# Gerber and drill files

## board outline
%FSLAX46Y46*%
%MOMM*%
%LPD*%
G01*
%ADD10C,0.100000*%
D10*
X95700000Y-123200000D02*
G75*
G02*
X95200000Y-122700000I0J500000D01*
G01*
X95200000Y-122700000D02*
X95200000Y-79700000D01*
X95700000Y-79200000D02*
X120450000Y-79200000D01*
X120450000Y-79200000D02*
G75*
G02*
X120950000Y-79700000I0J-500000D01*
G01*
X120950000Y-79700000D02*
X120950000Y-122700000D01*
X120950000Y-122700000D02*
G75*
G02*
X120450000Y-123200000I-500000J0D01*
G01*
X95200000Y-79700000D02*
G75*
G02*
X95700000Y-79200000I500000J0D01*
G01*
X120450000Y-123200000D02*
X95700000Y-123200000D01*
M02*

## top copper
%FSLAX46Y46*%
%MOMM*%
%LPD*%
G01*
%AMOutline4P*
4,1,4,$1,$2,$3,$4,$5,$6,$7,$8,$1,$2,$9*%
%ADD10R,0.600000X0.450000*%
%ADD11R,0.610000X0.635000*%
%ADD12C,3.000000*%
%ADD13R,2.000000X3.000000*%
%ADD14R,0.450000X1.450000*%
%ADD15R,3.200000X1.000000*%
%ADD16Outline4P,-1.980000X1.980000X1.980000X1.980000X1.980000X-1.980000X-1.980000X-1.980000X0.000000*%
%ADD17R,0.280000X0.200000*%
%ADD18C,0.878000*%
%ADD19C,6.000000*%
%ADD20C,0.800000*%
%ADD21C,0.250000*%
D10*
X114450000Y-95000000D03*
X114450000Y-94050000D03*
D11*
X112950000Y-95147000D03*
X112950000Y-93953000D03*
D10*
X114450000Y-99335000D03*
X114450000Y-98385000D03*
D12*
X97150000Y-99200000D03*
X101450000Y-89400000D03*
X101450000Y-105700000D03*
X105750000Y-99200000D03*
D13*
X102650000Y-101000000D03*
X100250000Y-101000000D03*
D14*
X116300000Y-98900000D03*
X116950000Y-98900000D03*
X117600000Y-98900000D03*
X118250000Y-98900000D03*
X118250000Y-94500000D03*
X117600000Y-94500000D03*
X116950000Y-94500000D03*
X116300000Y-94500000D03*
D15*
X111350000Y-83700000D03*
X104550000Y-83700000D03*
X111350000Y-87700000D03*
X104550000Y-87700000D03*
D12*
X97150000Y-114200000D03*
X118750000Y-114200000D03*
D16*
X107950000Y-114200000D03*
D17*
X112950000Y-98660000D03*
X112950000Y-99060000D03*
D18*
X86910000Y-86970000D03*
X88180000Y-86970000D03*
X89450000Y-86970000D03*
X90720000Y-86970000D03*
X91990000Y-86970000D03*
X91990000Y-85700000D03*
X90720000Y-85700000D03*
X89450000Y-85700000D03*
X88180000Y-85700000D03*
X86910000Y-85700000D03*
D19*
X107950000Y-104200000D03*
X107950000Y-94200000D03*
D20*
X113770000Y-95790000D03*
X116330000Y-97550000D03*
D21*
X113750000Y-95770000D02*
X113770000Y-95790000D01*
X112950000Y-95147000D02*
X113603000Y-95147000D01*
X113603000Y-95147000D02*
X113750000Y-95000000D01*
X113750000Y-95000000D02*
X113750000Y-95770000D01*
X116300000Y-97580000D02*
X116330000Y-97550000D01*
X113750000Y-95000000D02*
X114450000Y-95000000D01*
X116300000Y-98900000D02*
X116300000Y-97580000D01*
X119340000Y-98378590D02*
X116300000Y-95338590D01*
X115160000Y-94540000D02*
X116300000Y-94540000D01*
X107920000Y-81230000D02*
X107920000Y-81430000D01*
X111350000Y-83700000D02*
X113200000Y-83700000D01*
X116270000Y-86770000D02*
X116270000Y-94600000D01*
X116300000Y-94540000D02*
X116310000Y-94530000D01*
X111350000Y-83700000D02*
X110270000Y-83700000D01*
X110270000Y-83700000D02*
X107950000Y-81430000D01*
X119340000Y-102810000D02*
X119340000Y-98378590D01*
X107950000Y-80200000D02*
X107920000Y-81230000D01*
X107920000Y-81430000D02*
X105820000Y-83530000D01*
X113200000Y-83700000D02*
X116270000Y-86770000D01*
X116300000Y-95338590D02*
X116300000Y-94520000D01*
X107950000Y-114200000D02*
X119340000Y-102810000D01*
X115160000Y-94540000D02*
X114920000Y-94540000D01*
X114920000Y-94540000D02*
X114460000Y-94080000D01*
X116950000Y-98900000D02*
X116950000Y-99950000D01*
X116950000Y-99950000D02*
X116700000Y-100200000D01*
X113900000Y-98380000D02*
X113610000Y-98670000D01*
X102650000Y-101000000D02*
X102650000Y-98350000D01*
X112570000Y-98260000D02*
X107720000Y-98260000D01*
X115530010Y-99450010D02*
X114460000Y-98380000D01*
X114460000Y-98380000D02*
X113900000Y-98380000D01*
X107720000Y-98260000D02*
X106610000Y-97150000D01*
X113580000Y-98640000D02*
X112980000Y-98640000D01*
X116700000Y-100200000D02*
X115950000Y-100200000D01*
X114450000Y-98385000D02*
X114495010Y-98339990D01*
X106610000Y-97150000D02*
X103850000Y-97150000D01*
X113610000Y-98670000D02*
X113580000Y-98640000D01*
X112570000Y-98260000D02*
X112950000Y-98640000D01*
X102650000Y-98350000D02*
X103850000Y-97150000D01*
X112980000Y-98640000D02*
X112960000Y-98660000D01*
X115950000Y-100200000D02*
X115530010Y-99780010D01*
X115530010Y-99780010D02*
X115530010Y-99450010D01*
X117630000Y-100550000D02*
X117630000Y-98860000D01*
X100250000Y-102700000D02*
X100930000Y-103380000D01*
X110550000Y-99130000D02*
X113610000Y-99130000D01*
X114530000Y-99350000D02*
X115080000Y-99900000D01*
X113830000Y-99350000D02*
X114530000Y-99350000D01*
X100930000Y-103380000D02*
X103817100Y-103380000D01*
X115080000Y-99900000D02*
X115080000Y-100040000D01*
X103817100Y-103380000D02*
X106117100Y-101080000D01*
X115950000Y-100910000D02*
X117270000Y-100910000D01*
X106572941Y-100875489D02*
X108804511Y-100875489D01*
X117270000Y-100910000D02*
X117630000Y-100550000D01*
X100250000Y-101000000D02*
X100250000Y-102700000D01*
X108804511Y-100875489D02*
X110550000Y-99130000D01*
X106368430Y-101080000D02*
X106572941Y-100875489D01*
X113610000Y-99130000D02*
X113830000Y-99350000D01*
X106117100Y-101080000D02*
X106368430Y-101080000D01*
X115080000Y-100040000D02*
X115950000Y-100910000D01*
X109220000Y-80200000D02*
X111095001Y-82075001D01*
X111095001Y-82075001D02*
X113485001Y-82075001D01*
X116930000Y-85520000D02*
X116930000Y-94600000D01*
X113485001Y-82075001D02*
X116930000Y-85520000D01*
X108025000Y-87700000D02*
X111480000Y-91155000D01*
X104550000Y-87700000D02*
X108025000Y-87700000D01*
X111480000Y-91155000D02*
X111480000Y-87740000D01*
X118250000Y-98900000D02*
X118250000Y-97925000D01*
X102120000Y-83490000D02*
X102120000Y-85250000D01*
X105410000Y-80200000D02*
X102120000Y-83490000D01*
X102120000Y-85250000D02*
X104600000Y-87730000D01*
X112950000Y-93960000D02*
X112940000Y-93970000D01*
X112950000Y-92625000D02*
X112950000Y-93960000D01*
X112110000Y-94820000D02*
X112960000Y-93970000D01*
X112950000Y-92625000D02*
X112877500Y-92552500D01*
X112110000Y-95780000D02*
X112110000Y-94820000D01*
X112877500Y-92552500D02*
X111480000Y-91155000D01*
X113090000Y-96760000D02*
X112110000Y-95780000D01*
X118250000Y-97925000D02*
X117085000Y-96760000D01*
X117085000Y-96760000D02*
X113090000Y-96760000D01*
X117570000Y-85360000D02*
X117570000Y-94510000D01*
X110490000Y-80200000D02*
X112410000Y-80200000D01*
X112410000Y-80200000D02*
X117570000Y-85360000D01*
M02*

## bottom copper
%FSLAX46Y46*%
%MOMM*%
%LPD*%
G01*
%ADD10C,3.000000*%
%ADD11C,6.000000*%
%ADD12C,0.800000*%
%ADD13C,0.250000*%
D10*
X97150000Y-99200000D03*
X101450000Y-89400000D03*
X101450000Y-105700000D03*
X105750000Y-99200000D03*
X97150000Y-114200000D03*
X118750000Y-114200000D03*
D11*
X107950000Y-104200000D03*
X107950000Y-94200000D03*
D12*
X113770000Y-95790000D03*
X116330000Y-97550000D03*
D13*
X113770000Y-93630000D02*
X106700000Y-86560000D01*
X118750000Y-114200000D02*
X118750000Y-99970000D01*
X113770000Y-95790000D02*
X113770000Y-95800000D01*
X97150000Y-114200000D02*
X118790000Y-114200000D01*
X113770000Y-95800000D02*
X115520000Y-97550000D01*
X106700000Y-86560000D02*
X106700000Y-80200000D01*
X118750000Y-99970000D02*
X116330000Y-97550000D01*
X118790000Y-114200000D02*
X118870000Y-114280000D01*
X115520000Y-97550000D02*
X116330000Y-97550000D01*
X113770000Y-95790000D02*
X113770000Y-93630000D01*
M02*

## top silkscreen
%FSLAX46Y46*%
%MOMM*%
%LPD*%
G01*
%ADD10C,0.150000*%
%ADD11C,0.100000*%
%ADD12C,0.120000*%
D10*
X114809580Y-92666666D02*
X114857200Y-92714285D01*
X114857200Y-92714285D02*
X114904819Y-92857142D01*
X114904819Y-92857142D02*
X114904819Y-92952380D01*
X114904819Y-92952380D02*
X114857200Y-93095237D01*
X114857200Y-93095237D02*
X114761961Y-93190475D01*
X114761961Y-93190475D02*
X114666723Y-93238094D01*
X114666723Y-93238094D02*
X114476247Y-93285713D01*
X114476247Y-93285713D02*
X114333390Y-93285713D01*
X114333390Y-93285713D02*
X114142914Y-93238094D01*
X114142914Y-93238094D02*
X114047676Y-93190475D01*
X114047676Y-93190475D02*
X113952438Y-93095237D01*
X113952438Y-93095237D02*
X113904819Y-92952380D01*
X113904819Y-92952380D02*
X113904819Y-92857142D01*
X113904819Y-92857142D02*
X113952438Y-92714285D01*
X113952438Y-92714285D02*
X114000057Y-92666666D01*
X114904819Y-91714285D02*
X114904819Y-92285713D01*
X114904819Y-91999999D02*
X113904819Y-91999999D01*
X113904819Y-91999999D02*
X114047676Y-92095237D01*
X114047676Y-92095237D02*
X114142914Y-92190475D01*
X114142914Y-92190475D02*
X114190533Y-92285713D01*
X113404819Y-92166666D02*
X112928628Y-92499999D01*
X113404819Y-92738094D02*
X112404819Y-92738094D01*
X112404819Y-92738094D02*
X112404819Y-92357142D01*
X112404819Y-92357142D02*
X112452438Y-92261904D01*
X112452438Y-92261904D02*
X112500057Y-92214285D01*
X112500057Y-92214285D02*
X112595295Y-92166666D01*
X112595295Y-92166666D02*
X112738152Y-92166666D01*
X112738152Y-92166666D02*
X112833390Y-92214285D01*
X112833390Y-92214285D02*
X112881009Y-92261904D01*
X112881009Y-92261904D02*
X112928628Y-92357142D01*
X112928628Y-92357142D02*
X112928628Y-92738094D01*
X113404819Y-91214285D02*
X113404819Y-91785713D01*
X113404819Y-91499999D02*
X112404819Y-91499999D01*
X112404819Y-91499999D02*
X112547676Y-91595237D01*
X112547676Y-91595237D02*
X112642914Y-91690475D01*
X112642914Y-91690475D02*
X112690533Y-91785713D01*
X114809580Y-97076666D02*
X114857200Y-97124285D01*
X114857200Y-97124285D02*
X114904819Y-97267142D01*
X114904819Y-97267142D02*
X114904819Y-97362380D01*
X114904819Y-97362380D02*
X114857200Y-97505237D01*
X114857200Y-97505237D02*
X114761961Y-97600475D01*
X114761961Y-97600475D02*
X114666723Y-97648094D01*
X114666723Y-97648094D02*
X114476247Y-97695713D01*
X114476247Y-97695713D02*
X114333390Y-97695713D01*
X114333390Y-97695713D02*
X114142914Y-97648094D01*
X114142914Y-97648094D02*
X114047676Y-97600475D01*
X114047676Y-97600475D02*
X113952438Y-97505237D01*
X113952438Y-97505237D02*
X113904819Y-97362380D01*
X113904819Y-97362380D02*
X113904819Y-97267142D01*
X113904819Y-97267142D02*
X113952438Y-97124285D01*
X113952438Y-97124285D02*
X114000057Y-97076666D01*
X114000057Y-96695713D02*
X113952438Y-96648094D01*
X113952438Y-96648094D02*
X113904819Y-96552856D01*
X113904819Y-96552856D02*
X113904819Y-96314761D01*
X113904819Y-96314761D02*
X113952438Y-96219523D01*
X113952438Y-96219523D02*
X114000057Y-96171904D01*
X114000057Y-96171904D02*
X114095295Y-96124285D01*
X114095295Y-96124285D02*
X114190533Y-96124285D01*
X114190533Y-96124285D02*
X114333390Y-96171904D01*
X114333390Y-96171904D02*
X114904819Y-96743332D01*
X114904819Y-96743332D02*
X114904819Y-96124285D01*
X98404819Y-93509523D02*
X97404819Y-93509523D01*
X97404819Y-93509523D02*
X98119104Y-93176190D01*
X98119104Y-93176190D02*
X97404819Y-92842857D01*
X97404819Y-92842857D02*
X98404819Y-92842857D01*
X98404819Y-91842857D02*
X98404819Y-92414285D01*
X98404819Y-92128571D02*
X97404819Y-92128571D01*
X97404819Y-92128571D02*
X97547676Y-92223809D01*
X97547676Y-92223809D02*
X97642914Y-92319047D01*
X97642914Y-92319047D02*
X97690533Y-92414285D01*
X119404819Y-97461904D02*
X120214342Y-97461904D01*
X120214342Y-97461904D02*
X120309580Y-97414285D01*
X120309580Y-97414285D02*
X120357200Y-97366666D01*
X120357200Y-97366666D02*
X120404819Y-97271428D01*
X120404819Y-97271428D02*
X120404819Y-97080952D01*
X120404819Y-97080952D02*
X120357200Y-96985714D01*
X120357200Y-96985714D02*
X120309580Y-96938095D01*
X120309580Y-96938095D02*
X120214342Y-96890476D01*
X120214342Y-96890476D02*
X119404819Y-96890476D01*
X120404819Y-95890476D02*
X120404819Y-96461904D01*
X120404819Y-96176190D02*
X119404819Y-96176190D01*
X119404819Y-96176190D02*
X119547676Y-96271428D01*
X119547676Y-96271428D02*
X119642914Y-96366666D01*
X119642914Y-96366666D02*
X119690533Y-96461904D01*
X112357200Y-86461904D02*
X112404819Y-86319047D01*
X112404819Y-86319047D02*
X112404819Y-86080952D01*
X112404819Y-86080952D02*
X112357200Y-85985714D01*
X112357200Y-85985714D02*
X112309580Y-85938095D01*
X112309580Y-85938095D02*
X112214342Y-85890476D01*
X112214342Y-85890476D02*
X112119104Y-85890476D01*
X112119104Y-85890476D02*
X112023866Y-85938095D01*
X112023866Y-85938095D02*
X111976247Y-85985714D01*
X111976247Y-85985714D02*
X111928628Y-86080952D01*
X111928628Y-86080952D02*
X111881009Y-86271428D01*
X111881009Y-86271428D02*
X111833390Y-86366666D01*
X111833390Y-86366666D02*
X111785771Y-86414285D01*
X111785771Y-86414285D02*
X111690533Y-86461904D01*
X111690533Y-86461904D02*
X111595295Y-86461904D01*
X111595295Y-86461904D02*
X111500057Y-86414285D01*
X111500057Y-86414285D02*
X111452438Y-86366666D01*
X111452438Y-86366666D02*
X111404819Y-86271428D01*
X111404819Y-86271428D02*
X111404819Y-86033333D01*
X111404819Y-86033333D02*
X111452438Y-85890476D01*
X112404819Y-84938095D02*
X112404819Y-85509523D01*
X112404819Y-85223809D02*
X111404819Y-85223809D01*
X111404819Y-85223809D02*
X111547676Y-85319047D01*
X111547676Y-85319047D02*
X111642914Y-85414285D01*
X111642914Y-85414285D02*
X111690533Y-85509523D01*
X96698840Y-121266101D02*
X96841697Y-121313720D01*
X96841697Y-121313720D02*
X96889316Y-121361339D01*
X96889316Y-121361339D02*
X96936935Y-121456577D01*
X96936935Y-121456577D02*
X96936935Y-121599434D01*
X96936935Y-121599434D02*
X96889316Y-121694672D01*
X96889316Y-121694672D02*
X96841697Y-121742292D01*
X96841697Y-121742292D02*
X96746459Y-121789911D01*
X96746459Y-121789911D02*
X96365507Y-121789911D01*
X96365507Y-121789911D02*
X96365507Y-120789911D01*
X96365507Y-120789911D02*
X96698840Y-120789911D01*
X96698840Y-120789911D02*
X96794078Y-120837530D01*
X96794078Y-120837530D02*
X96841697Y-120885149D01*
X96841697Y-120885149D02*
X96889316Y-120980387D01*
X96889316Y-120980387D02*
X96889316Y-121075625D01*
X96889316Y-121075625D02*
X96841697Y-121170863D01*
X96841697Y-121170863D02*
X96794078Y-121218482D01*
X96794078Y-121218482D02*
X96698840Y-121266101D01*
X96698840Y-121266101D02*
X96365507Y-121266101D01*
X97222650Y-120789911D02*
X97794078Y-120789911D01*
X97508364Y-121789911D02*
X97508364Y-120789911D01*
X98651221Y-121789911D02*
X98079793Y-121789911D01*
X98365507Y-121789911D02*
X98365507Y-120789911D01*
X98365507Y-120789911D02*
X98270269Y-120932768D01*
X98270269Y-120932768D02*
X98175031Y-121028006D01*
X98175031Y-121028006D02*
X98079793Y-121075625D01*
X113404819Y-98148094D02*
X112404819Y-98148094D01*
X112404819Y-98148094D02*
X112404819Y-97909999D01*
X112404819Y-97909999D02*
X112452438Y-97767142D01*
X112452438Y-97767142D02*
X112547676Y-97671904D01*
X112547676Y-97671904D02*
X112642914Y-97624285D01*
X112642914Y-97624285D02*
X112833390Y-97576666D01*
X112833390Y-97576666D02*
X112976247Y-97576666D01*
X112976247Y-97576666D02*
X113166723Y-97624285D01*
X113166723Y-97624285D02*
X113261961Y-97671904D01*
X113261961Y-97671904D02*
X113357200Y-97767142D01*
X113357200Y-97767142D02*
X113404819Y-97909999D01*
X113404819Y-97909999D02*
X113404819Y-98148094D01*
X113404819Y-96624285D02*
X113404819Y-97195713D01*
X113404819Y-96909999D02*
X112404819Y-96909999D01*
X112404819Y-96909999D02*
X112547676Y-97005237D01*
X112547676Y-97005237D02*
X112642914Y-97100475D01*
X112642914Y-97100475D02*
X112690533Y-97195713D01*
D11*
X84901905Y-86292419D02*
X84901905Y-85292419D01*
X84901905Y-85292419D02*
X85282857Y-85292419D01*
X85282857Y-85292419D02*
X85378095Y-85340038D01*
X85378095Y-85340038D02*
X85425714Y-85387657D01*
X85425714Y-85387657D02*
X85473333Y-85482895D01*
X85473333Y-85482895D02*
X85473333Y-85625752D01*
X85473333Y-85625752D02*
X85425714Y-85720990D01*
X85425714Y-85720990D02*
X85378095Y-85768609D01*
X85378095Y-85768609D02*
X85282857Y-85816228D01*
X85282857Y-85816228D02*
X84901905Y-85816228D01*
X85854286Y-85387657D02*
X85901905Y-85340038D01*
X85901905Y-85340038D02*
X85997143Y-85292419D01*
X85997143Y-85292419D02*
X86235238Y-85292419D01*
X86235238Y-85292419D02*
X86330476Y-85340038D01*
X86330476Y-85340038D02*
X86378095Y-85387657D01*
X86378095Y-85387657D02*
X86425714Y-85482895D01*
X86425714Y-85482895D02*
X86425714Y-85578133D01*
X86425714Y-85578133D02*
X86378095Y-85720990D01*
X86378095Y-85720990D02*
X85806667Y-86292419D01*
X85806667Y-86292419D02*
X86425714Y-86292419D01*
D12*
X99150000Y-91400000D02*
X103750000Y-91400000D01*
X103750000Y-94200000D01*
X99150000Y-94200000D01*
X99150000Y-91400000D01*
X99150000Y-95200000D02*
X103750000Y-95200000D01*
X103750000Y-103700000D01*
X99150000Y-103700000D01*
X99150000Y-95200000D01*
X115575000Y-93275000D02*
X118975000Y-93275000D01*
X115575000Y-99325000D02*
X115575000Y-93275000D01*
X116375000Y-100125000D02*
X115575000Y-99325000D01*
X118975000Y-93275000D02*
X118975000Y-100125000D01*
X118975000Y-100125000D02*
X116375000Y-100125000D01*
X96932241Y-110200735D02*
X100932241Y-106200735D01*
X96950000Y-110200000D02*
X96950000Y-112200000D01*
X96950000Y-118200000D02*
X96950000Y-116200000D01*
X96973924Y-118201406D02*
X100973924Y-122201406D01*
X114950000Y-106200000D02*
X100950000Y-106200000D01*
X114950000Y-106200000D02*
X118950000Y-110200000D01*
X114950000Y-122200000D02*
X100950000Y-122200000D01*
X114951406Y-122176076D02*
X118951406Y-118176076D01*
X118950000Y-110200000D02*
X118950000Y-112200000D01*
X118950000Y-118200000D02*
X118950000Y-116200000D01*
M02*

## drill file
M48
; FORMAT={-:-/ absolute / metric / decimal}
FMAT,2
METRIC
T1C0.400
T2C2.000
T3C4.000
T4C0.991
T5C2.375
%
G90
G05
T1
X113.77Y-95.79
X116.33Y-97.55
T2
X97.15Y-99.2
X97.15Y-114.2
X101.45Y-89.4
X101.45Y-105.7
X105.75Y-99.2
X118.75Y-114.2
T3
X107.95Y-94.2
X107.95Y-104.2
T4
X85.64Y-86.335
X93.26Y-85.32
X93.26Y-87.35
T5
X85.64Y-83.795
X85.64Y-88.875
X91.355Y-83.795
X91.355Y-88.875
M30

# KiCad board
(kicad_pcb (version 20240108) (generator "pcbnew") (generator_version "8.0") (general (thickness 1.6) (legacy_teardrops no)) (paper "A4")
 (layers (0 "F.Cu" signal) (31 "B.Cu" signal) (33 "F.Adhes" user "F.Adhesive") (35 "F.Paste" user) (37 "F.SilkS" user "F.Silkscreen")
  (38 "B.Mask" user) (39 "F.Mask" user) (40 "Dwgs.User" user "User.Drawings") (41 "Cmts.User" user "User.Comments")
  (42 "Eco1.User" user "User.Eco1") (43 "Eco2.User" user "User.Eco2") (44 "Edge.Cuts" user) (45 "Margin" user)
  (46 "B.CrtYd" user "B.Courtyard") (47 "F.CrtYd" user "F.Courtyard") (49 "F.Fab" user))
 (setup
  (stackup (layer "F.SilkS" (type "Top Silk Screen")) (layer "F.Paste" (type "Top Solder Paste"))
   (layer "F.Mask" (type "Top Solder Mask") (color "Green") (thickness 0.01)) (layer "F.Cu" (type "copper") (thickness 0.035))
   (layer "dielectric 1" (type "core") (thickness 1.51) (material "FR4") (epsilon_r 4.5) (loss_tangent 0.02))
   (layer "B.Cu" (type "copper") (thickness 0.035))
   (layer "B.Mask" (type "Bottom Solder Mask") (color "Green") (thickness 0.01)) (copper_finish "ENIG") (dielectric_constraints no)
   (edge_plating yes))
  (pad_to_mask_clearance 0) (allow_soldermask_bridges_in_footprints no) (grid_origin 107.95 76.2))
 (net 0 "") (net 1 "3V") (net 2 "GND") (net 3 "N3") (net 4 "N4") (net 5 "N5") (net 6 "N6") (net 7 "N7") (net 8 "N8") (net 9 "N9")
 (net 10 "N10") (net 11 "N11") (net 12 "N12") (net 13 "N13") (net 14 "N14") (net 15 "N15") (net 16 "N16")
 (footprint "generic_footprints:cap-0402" (layer "F.Cu") (at 114.45 94.525 90)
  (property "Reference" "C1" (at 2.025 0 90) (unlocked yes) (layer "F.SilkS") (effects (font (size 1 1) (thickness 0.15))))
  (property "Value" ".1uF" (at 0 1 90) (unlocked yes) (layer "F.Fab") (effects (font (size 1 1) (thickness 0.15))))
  (pad "1" smd rect (at -0.475 0 90) (size 0.45 0.6) (layers "F.Cu" "F.Paste" "F.Mask") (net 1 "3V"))
  (pad "2" smd rect (at 0.475 0 90) (size 0.45 0.6) (layers "F.Cu" "F.Paste" "F.Mask") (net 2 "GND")))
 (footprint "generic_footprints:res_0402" (layer "F.Cu") (at 112.95 94.55 90)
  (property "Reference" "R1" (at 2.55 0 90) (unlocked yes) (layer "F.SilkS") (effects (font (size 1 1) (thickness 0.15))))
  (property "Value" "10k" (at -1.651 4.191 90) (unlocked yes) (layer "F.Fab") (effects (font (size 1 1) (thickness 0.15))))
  (pad "1" smd rect (at -0.597 0 90) (size 0.635 0.61) (layers "F.Cu" "F.Paste" "F.Mask") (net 1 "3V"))
  (pad "2" smd rect (at 0.597 0 90) (size 0.635 0.61) (layers "F.Cu" "F.Paste" "F.Mask") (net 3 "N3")))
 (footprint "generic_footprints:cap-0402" (layer "F.Cu") (at 114.45 98.86 90)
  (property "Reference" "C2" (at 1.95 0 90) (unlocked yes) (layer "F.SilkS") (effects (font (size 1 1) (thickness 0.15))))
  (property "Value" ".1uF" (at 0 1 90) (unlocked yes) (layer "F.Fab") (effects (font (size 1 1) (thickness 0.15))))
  (pad "1" smd rect (at -0.475 0 90) (size 0.45 0.6) (layers "F.Cu" "F.Paste" "F.Mask") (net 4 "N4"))
  (pad "2" smd rect (at 0.475 0 90) (size 0.45 0.6) (layers "F.Cu" "F.Paste" "F.Mask") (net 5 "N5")))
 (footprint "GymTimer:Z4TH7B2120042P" (layer "F.Cu") (at 101.45 95.2)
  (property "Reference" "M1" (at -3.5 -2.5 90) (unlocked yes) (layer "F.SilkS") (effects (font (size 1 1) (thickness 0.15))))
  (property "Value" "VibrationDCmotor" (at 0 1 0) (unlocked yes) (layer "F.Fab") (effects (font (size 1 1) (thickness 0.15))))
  (fp_rect (start -2.3 -3.8) (end 2.3 -1) (stroke (width 0.12) (type solid)) (fill none) (layer "F.SilkS"))
  (fp_rect (start -2.3 0) (end 2.3 8.5) (stroke (width 0.12) (type solid)) (fill none) (layer "F.SilkS"))
  (pad "" thru_hole circle (at -4.3 4) (size 3 3) (drill 2) (layers "*.Cu" "*.Mask") (remove_unused_layers no))
  (pad "" thru_hole circle (at 0 -5.8) (size 3 3) (drill 2) (layers "*.Cu" "*.Mask") (remove_unused_layers no))
  (pad "" thru_hole circle (at 0 10.5) (size 3 3) (drill 2) (layers "*.Cu" "*.Mask") (remove_unused_layers no))
  (pad "" thru_hole circle (at 4.3 4) (size 3 3) (drill 2) (layers "*.Cu" "*.Mask") (remove_unused_layers no))
  (pad "1" smd rect (at 1.2 5.8) (size 2 3) (layers "F.Cu" "F.Paste" "F.Mask") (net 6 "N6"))
  (pad "2" smd rect (at -1.2 5.8) (size 2 3) (layers "F.Cu" "F.Paste" "F.Mask") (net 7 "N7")))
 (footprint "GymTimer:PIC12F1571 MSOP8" (layer "F.Cu") (at 117.275 96.7 90)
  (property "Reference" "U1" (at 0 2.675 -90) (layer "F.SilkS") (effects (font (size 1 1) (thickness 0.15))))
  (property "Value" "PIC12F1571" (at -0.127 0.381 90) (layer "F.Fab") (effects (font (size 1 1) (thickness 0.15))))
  (fp_line (start 3.425 -1.7) (end 3.425 1.7) (stroke (width 0.12) (type solid)) (layer "F.SilkS"))
  (fp_line (start -2.625 -1.7) (end 3.425 -1.7) (stroke (width 0.12) (type solid)) (layer "F.SilkS"))
  (fp_line (start -3.425 -0.9) (end -2.625 -1.7) (stroke (width 0.12) (type solid)) (layer "F.SilkS"))
  (fp_line (start 3.425 1.7) (end -3.425 1.7) (stroke (width 0.12) (type solid)) (layer "F.SilkS"))
  (fp_line (start -3.425 1.7) (end -3.425 -0.9) (stroke (width 0.12) (type solid)) (layer "F.SilkS"))
  (pad "1" smd rect (at -2.2 -0.975) (size 0.45 1.45) (layers "F.Cu" "F.Paste" "F.Mask") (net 1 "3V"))
  (pad "2" smd rect (at -2.2 -0.325) (size 0.45 1.45) (layers "F.Cu" "F.Paste" "F.Mask") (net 6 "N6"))
  (pad "3" smd rect (at -2.2 0.325) (size 0.45 1.45) (layers "F.Cu" "F.Paste" "F.Mask") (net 7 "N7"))
  (pad "4" smd rect (at -2.2 0.975) (size 0.45 1.45) (layers "F.Cu" "F.Paste" "F.Mask") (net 3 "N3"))
  (pad "5" smd rect (at 2.2 0.975) (size 0.45 1.45) (layers "F.Cu" "F.Paste" "F.Mask") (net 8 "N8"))
  (pad "6" smd rect (at 2.2 0.325) (size 0.45 1.45) (layers "F.Cu" "F.Paste" "F.Mask") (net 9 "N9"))
  (pad "7" smd rect (at 2.2 -0.325) (size 0.45 1.45) (layers "F.Cu" "F.Paste" "F.Mask") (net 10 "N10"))
  (pad "8" smd rect (at 2.2 -0.975) (size 0.45 1.45) (layers "F.Cu" "F.Paste" "F.Mask") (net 2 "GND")))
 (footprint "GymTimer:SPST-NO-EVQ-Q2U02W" (layer "F.Cu") (at 107.95 85.7 180)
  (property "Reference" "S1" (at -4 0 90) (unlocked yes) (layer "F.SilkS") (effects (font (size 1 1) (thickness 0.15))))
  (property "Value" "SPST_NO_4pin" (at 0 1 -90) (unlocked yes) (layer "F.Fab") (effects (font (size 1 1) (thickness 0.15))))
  (pad "1" smd rect (at -3.4 2 180) (size 3.2 1) (layers "F.Cu" "F.Paste" "F.Mask") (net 2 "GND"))
  (pad "2" smd rect (at 3.4 2 180) (size 3.2 1) (layers "F.Cu" "F.Paste" "F.Mask") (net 2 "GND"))
  (pad "3" smd rect (at -3.4 -2 180) (size 3.2 1) (layers "F.Cu" "F.Paste" "F.Mask") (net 3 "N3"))
  (pad "4" smd rect (at 3.4 -2 180) (size 3.2 1) (layers "F.Cu" "F.Paste" "F.Mask") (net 3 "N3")))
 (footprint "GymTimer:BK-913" (layer "F.Cu") (at 107.95 114.2)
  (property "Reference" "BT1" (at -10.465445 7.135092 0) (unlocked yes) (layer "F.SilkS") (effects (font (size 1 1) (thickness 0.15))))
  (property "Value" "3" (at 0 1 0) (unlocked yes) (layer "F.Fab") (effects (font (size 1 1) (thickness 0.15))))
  (fp_line (start -11.017759 -3.999265) (end -7.017759 -7.999265) (stroke (width 0.12) (type solid)) (layer "F.SilkS"))
  (fp_line (start -11 -4) (end -11 -2) (stroke (width 0.12) (type solid)) (layer "F.SilkS"))
  (fp_line (start -11 4) (end -11 2) (stroke (width 0.12) (type solid)) (layer "F.SilkS"))
  (fp_line (start -10.976076 4.001406) (end -6.976076 8.001406) (stroke (width 0.12) (type solid)) (layer "F.SilkS"))
  (fp_line (start 7 -8) (end -7 -8) (stroke (width 0.12) (type solid)) (layer "F.SilkS"))
  (fp_line (start 7 -8) (end 11 -4) (stroke (width 0.12) (type solid)) (layer "F.SilkS"))
  (fp_line (start 7 8) (end -7 8) (stroke (width 0.12) (type solid)) (layer "F.SilkS"))
  (fp_line (start 7.001406 7.976076) (end 11.001406 3.976076) (stroke (width 0.12) (type solid)) (layer "F.SilkS"))
  (fp_line (start 11 -4) (end 11 -2) (stroke (width 0.12) (type solid)) (layer "F.SilkS"))
  (fp_line (start 11 4) (end 11 2) (stroke (width 0.12) (type solid)) (layer "F.SilkS"))
  (pad "1" thru_hole circle (at -10.8 0) (size 3 3) (drill 2) (layers "*.Cu" "*.Mask") (remove_unused_layers no) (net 1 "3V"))
  (pad "1" thru_hole circle (at 10.8 0) (size 3 3) (drill 2) (layers "*.Cu" "*.Mask") (remove_unused_layers no) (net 1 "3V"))
  (pad "2" smd roundrect (at 0 0) (size 3.96 3.96) (layers "F.Cu" "F.Paste" "F.Mask") (roundrect_rratio 0.25) (chamfer_ratio 0)
   (chamfer top_left top_right bottom_left bottom_right) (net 2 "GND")))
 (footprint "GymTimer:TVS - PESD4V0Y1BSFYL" (layer "F.Cu") (at 112.95 98.86 -90)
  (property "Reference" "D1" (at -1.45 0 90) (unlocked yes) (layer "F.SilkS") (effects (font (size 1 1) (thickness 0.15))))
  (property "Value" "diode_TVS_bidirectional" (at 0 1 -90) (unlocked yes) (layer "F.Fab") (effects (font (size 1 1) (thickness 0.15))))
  (pad "1" smd rect (at -0.2 0 270) (size 0.2 0.28) (layers "F.Cu" "F.Paste" "F.Mask") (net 5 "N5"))
  (pad "2" smd rect (at 0.2 0 270) (size 0.2 0.28) (layers "F.Cu" "F.Paste" "F.Mask") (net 4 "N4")))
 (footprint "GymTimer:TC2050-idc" (layer "F.Cu") (at 85.64 86.335)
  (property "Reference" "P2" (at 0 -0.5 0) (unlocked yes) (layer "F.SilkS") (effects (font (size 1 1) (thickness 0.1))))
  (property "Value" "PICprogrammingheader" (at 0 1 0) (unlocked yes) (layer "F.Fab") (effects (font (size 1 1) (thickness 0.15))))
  (pad "" np_thru_hole circle (at 0 -2.54) (size 2.3749 2.3749) (drill 2.3749) (layers "F&B.Cu" "*.Mask"))
  (pad "" np_thru_hole circle (at 0 0) (size 0.9906 0.9906) (drill 0.9906) (layers "F&B.Cu" "*.Mask"))
  (pad "" np_thru_hole circle (at 0 2.54) (size 2.3749 2.3749) (drill 2.3749) (layers "F&B.Cu" "*.Mask"))
  (pad "" np_thru_hole circle (at 5.715 -2.54) (size 2.3749 2.3749) (drill 2.3749) (layers "F&B.Cu" "*.Mask"))
  (pad "" np_thru_hole circle (at 5.715 2.54) (size 2.3749 2.3749) (drill 2.3749) (layers "F&B.Cu" "*.Mask"))
  (pad "" np_thru_hole circle (at 7.62 -1.015) (size 0.9906 0.9906) (drill 0.9906) (layers "F&B.Cu" "*.Mask"))
  (pad "" np_thru_hole circle (at 7.62 1.015) (size 0.9906 0.9906) (drill 0.9906) (layers "F&B.Cu" "*.Mask"))
  (pad "1" smd circle (at 1.27 0.635) (size 0.878 0.878) (layers "F.Cu" "F.Paste" "F.Mask") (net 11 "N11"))
  (pad "2" smd circle (at 2.54 0.635) (size 0.878 0.878) (layers "F.Cu" "F.Paste" "F.Mask") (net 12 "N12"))
  (pad "3" smd circle (at 3.81 0.635) (size 0.878 0.878) (layers "F.Cu" "F.Paste" "F.Mask") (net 10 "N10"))
  (pad "4" smd circle (at 5.08 0.635) (size 0.878 0.878) (layers "F.Cu" "F.Paste" "F.Mask") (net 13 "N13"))
  (pad "5" smd circle (at 6.35 0.635) (size 0.878 0.878) (layers "F.Cu" "F.Paste" "F.Mask") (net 2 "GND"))
  (pad "6" smd circle (at 6.35 -0.635) (size 0.878 0.878) (layers "F.Cu" "F.Paste" "F.Mask") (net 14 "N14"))
  (pad "7" smd circle (at 5.08 -0.635) (size 0.878 0.878) (layers "F.Cu" "F.Paste" "F.Mask") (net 1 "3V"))
  (pad "8" smd circle (at 3.81 -0.635) (size 0.878 0.878) (layers "F.Cu" "F.Paste" "F.Mask") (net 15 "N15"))
  (pad "9" smd circle (at 2.54 -0.635) (size 0.878 0.878) (layers "F.Cu" "F.Paste" "F.Mask") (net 3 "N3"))
  (pad "10" smd circle (at 1.27 -0.635) (size 0.878 0.878) (layers "F.Cu" "F.Paste" "F.Mask") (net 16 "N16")))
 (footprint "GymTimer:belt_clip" (layer "B.Cu") (at 107.95 99.2 180)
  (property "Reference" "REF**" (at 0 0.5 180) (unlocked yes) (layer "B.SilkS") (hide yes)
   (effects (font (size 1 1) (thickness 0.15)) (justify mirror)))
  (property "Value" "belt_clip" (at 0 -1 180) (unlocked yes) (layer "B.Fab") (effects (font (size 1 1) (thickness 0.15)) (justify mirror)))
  (pad "1" thru_hole circle (at 0 -5 180) (size 6 6) (drill 4) (layers "*.Cu" "*.Mask") (remove_unused_layers no))
  (pad "1" thru_hole circle (at 0 5 180) (size 6 6) (drill 4) (layers "*.Cu" "*.Mask") (remove_unused_layers no)))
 (gr_arc (start 95.7 123.2) (mid 95.346447 123.053553) (end 95.2 122.7) (stroke (width 0.1) (type solid)) (layer "Edge.Cuts"))
 (gr_line (start 95.2 122.7) (end 95.2 79.7) (stroke (width 0.1) (type solid)) (layer "Edge.Cuts"))
 (gr_line (start 95.7 79.2) (end 120.45 79.2) (stroke (width 0.1) (type solid)) (layer "Edge.Cuts"))
 (gr_arc (start 120.45 79.2) (mid 120.803553 79.346447) (end 120.95 79.7) (stroke (width 0.1) (type solid)) (layer "Edge.Cuts"))
 (gr_line (start 120.95 79.7) (end 120.95 122.7) (stroke (width 0.1) (type solid)) (layer "Edge.Cuts"))
 (gr_arc (start 120.95 122.7) (mid 120.803553 123.053553) (end 120.45 123.2) (stroke (width 0.1) (type solid)) (layer "Edge.Cuts"))
 (gr_arc (start 95.2 79.7) (mid 95.346447 79.346447) (end 95.7 79.2) (stroke (width 0.1) (type solid)) (layer "Edge.Cuts"))
 (gr_line (start 120.45 123.2) (end 95.7 123.2) (stroke (width 0.1) (type solid)) (layer "Edge.Cuts"))
 (segment (start 113.75 95.77) (end 113.77 95.79) (width 0.25) (layer "F.Cu") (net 1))
 (segment (start 112.95 95.147) (end 113.603 95.147) (width 0.25) (layer "F.Cu") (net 1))
 (segment (start 113.603 95.147) (end 113.75 95) (width 0.25) (layer "F.Cu") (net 1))
 (segment (start 113.75 95) (end 113.75 95.77) (width 0.25) (layer "F.Cu") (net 1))
 (segment (start 116.3 97.58) (end 116.33 97.55) (width 0.25) (layer "F.Cu") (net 1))
 (segment (start 113.75 95) (end 114.45 95) (width 0.25) (layer "F.Cu") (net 1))
 (segment (start 116.3 98.9) (end 116.3 97.58) (width 0.25) (layer "F.Cu") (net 1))
 (via (at 113.77 95.79) (size 0.8) (drill 0.4) (layers "F.Cu" "B.Cu") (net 1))
 (via (at 116.33 97.55) (size 0.8) (drill 0.4) (layers "F.Cu" "B.Cu") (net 1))
 (segment (start 113.77 93.63) (end 106.7 86.56) (width 0.25) (layer "B.Cu") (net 1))
 (segment (start 118.75 114.2) (end 118.75 99.97) (width 0.25) (layer "B.Cu") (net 1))
 (segment (start 113.77 95.79) (end 113.77 95.8) (width 0.25) (layer "B.Cu") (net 1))
 (segment (start 97.15 114.2) (end 118.79 114.2) (width 0.25) (layer "B.Cu") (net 1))
 (segment (start 113.77 95.8) (end 115.52 97.55) (width 0.25) (layer "B.Cu") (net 1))
 (segment (start 106.7 86.56) (end 106.7 80.2) (width 0.25) (layer "B.Cu") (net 1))
 (segment (start 118.75 99.97) (end 116.33 97.55) (width 0.25) (layer "B.Cu") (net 1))
 (segment (start 118.79 114.2) (end 118.87 114.28) (width 0.25) (layer "B.Cu") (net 1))
 (segment (start 115.52 97.55) (end 116.33 97.55) (width 0.25) (layer "B.Cu") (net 1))
 (segment (start 113.77 95.79) (end 113.77 93.63) (width 0.25) (layer "B.Cu") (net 1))
 (segment (start 119.34 98.37859) (end 116.3 95.33859) (width 0.25) (layer "F.Cu") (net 2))
 (segment (start 115.16 94.54) (end 116.3 94.54) (width 0.25) (layer "F.Cu") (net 2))
 (segment (start 107.92 81.23) (end 107.92 81.43) (width 0.25) (layer "F.Cu") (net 2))
 (segment (start 111.35 83.7) (end 113.2 83.7) (width 0.25) (layer "F.Cu") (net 2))
 (segment (start 116.27 86.77) (end 116.27 94.6) (width 0.25) (layer "F.Cu") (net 2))
 (segment (start 116.3 94.54) (end 116.31 94.53) (width 0.25) (layer "F.Cu") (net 2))
 (segment (start 111.35 83.7) (end 110.27 83.7) (width 0.25) (layer "F.Cu") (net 2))
 (segment (start 110.27 83.7) (end 107.95 81.43) (width 0.25) (layer "F.Cu") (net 2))
 (segment (start 119.34 102.81) (end 119.34 98.37859) (width 0.25) (layer "F.Cu") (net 2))
 (segment (start 107.95 80.2) (end 107.92 81.23) (width 0.25) (layer "F.Cu") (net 2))
 (segment (start 107.92 81.43) (end 105.82 83.53) (width 0.25) (layer "F.Cu") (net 2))
 (segment (start 113.2 83.7) (end 116.27 86.77) (width 0.25) (layer "F.Cu") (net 2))
 (segment (start 116.3 95.33859) (end 116.3 94.52) (width 0.25) (layer "F.Cu") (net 2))
 (segment (start 107.95 114.2) (end 119.34 102.81) (width 0.25) (layer "F.Cu") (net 2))
 (segment (start 115.16 94.54) (end 114.92 94.54) (width 0.25) (layer "F.Cu") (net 2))
 (segment (start 114.92 94.54) (end 114.46 94.08) (width 0.25) (layer "F.Cu") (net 2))
 (segment (start 116.95 98.9) (end 116.95 99.95) (width 0.25) (layer "F.Cu") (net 5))
 (segment (start 116.95 99.95) (end 116.7 100.2) (width 0.25) (layer "F.Cu") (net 5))
 (segment (start 113.9 98.38) (end 113.61 98.67) (width 0.25) (layer "F.Cu") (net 5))
 (segment (start 102.65 101) (end 102.65 98.35) (width 0.25) (layer "F.Cu") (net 5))
 (segment (start 112.57 98.26) (end 107.72 98.26) (width 0.25) (layer "F.Cu") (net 5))
 (segment (start 115.53001 99.45001) (end 114.46 98.38) (width 0.25) (layer "F.Cu") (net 5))
 (segment (start 114.46 98.38) (end 113.9 98.38) (width 0.25) (layer "F.Cu") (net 5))
 (segment (start 107.72 98.26) (end 106.61 97.15) (width 0.25) (layer "F.Cu") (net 5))
 (segment (start 113.58 98.64) (end 112.98 98.64) (width 0.25) (layer "F.Cu") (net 5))
 (segment (start 116.7 100.2) (end 115.95 100.2) (width 0.25) (layer "F.Cu") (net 5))
 (segment (start 114.45 98.385) (end 114.49501 98.33999) (width 0.25) (layer "F.Cu") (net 5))
 (segment (start 106.61 97.15) (end 103.85 97.15) (width 0.25) (layer "F.Cu") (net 5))
 (segment (start 113.61 98.67) (end 113.58 98.64) (width 0.25) (layer "F.Cu") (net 5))
 (segment (start 112.57 98.26) (end 112.95 98.64) (width 0.25) (layer "F.Cu") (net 5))
 (segment (start 102.65 98.35) (end 103.85 97.15) (width 0.25) (layer "F.Cu") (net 5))
 (segment (start 112.98 98.64) (end 112.96 98.66) (width 0.25) (layer "F.Cu") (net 5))
 (segment (start 115.95 100.2) (end 115.53001 99.78001) (width 0.25) (layer "F.Cu") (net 5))
 (segment (start 115.53001 99.78001) (end 115.53001 99.45001) (width 0.25) (layer "F.Cu") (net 5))
 (segment (start 117.63 100.55) (end 117.63 98.86) (width 0.25) (layer "F.Cu") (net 4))
 (segment (start 100.25 102.7) (end 100.93 103.38) (width 0.25) (layer "F.Cu") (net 4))
 (segment (start 110.55 99.13) (end 113.61 99.13) (width 0.25) (layer "F.Cu") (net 4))
 (segment (start 114.53 99.35) (end 115.08 99.9) (width 0.25) (layer "F.Cu") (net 4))
 (segment (start 113.83 99.35) (end 114.53 99.35) (width 0.25) (layer "F.Cu") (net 4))
 (segment (start 100.93 103.38) (end 103.8171 103.38) (width 0.25) (layer "F.Cu") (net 4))
 (segment (start 115.08 99.9) (end 115.08 100.04) (width 0.25) (layer "F.Cu") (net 4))
 (segment (start 103.8171 103.38) (end 106.1171 101.08) (width 0.25) (layer "F.Cu") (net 4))
 (segment (start 115.95 100.91) (end 117.27 100.91) (width 0.25) (layer "F.Cu") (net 4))
 (segment (start 106.572941 100.875489) (end 108.804511 100.875489) (width 0.25) (layer "F.Cu") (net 4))
 (segment (start 117.27 100.91) (end 117.63 100.55) (width 0.25) (layer "F.Cu") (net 4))
 (segment (start 100.25 101) (end 100.25 102.7) (width 0.25) (layer "F.Cu") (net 4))
 (segment (start 108.804511 100.875489) (end 110.55 99.13) (width 0.25) (layer "F.Cu") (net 4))
 (segment (start 106.36843 101.08) (end 106.572941 100.875489) (width 0.25) (layer "F.Cu") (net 4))
 (segment (start 113.61 99.13) (end 113.83 99.35) (width 0.25) (layer "F.Cu") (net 4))
 (segment (start 106.1171 101.08) (end 106.36843 101.08) (width 0.25) (layer "F.Cu") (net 4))
 (segment (start 115.08 100.04) (end 115.95 100.91) (width 0.25) (layer "F.Cu") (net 4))
 (segment (start 109.22 80.2) (end 111.095001 82.075001) (width 0.25) (layer "F.Cu") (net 10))
 (segment (start 111.095001 82.075001) (end 113.485001 82.075001) (width 0.25) (layer "F.Cu") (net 10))
 (segment (start 116.93 85.52) (end 116.93 94.6) (width 0.25) (layer "F.Cu") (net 10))
 (segment (start 113.485001 82.075001) (end 116.93 85.52) (width 0.25) (layer "F.Cu") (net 10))
 (segment (start 108.025 87.7) (end 111.48 91.155) (width 0.25) (layer "F.Cu") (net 3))
 (segment (start 104.55 87.7) (end 108.025 87.7) (width 0.25) (layer "F.Cu") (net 3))
 (segment (start 111.48 91.155) (end 111.48 87.74) (width 0.25) (layer "F.Cu") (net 3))
 (segment (start 118.25 98.9) (end 118.25 97.925) (width 0.25) (layer "F.Cu") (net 3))
 (segment (start 102.12 83.49) (end 102.12 85.25) (width 0.25) (layer "F.Cu") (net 3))
 (segment (start 105.41 80.2) (end 102.12 83.49) (width 0.25) (layer "F.Cu") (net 3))
 (segment (start 102.12 85.25) (end 104.6 87.73) (width 0.25) (layer "F.Cu") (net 3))
 (segment (start 112.95 93.96) (end 112.94 93.97) (width 0.25) (layer "F.Cu") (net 3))
 (segment (start 112.95 92.625) (end 112.95 93.96) (width 0.25) (layer "F.Cu") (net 3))
 (segment (start 112.11 94.82) (end 112.96 93.97) (width 0.25) (layer "F.Cu") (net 3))
 (segment (start 112.95 92.625) (end 112.8775 92.5525) (width 0.25) (layer "F.Cu") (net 3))
 (segment (start 112.11 95.78) (end 112.11 94.82) (width 0.25) (layer "F.Cu") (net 3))
 (segment (start 112.8775 92.5525) (end 111.48 91.155) (width 0.25) (layer "F.Cu") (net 3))
 (segment (start 113.09 96.76) (end 112.11 95.78) (width 0.25) (layer "F.Cu") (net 3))
 (segment (start 118.25 97.925) (end 117.085 96.76) (width 0.25) (layer "F.Cu") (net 3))
 (segment (start 117.085 96.76) (end 113.09 96.76) (width 0.25) (layer "F.Cu") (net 3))
 (segment (start 117.57 85.36) (end 117.57 94.51) (width 0.25) (layer "F.Cu") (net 9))
 (segment (start 110.49 80.2) (end 112.41 80.2) (width 0.25) (layer "F.Cu") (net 9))
 (segment (start 112.41 80.2) (end 117.57 85.36) (width 0.25) (layer "F.Cu") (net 9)))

